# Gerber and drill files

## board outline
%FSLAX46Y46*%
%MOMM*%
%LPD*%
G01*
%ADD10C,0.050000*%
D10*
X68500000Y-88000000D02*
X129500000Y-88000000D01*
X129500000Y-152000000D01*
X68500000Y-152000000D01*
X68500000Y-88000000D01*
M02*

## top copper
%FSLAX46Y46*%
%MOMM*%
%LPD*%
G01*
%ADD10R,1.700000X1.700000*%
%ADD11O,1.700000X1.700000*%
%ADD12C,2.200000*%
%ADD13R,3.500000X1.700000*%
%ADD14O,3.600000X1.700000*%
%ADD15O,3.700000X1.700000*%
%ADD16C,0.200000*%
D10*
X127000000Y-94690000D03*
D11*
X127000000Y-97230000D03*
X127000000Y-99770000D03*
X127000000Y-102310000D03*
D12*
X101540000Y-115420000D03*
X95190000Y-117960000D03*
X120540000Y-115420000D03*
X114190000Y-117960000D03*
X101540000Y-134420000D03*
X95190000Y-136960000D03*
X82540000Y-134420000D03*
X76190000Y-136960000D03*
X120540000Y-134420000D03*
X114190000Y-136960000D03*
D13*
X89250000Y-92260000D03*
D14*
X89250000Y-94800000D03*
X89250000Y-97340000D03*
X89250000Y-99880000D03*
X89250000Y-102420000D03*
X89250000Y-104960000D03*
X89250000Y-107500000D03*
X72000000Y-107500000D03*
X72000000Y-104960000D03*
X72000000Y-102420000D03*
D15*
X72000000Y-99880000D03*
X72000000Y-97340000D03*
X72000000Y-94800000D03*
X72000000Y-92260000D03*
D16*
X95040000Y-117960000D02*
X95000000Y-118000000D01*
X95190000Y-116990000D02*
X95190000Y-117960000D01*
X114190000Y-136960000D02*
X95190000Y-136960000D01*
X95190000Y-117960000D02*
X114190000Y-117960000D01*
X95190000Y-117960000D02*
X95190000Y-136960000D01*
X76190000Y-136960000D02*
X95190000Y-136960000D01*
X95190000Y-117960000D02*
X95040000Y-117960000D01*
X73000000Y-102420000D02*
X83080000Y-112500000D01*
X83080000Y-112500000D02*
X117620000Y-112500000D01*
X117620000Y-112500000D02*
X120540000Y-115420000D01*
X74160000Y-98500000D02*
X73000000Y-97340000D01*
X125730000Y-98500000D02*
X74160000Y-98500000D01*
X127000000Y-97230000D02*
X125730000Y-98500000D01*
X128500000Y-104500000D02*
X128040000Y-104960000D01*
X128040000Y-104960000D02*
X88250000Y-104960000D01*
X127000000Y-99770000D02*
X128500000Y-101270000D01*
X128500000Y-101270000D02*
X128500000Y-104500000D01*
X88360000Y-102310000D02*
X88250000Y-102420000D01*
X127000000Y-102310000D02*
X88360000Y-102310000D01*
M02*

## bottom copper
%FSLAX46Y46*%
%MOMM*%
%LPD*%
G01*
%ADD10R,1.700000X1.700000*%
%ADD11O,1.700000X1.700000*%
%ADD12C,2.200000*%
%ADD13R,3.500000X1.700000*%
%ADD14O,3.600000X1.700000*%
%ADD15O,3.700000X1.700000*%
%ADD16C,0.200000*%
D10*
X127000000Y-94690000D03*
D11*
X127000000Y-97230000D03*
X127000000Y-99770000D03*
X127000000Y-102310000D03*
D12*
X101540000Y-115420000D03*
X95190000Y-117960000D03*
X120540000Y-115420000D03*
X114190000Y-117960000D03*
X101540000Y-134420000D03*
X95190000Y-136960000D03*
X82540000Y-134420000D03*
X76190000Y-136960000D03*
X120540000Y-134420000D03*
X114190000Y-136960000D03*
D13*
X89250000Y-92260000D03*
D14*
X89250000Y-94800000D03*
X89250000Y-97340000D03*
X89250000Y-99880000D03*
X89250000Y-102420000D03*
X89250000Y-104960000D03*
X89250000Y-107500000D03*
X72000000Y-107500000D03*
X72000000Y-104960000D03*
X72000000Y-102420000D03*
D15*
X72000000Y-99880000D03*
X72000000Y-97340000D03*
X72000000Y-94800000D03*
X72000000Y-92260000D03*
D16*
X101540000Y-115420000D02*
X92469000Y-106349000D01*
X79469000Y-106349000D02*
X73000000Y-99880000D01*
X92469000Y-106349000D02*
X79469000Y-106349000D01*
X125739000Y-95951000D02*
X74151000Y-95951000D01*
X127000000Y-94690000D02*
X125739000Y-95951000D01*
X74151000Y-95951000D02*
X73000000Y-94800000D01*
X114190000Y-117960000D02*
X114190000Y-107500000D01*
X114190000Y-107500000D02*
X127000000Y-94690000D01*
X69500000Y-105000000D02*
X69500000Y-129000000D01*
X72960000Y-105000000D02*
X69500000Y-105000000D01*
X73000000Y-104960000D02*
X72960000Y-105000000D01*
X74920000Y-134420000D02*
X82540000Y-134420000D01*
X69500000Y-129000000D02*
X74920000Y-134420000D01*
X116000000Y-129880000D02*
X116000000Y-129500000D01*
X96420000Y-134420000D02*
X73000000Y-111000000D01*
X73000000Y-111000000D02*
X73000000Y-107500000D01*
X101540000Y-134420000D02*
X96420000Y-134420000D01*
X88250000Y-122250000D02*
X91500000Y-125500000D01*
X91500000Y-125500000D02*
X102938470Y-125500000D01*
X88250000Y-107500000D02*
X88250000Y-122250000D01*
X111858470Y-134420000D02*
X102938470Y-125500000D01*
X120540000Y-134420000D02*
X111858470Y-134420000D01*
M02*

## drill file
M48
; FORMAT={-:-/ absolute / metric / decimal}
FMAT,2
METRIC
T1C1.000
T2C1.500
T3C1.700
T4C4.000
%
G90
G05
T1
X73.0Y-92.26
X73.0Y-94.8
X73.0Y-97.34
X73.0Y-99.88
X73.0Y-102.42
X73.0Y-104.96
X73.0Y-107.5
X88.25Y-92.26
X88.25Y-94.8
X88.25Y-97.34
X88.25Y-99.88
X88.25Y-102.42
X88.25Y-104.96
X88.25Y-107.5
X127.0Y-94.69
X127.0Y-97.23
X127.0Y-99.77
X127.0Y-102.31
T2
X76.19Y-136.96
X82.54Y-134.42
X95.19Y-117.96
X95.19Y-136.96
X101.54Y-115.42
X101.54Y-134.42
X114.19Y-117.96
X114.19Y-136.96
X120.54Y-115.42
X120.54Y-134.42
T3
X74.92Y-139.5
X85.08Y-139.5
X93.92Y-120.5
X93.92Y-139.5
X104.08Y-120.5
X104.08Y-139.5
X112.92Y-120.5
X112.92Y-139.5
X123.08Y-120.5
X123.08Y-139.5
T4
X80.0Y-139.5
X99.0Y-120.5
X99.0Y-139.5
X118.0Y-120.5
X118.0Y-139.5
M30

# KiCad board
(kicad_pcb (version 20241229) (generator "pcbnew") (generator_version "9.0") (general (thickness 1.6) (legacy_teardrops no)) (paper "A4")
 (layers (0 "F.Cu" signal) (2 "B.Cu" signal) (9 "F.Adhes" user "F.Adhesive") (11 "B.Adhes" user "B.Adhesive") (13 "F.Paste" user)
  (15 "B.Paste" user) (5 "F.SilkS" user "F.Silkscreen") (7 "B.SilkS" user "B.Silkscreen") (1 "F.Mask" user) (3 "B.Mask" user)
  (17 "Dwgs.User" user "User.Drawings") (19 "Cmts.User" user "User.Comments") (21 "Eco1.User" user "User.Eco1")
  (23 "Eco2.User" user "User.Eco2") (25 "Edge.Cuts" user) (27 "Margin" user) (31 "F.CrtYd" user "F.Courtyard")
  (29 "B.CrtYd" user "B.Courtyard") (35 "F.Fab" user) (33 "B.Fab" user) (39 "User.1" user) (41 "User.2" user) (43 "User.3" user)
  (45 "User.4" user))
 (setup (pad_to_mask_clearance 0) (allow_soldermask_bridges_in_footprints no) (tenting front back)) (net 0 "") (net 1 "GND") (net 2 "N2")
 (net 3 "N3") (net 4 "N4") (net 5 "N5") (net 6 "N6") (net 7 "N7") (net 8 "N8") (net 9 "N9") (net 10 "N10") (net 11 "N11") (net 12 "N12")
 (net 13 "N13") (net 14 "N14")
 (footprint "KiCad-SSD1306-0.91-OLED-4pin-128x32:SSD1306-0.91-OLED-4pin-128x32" (layer "F.Cu") (at 90.5 92.5)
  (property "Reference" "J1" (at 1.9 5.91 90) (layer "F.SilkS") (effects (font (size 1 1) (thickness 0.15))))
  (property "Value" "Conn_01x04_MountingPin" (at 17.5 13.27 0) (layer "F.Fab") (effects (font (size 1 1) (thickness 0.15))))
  (pad "1" thru_hole rect (at 36.5 2.19) (size 1.7 1.7) (drill 1) (layers "*.Cu" "*.Mask") (remove_unused_layers no) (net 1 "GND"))
  (pad "2" thru_hole oval (at 36.5 4.73) (size 1.7 1.7) (drill 1) (layers "*.Cu" "*.Mask") (remove_unused_layers no) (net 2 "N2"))
  (pad "3" thru_hole oval (at 36.5 7.27) (size 1.7 1.7) (drill 1) (layers "*.Cu" "*.Mask") (remove_unused_layers no) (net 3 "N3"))
  (pad "4" thru_hole oval (at 36.5 9.81) (size 1.7 1.7) (drill 1) (layers "*.Cu" "*.Mask") (remove_unused_layers no) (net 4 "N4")))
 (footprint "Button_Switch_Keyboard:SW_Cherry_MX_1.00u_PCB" (layer "F.Cu") (at 101.54 115.42)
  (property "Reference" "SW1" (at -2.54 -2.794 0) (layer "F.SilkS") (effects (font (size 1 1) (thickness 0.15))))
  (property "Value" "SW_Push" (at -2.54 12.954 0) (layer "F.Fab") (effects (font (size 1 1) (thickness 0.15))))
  (pad "" np_thru_hole circle (at -7.62 5.08) (size 1.7 1.7) (drill 1.7) (layers "*.Cu" "*.Mask"))
  (pad "" np_thru_hole circle (at -2.54 5.08) (size 4 4) (drill 4) (layers "*.Cu" "*.Mask"))
  (pad "" np_thru_hole circle (at 2.54 5.08) (size 1.7 1.7) (drill 1.7) (layers "*.Cu" "*.Mask"))
  (pad "1" thru_hole circle (at 0 0) (size 2.2 2.2) (drill 1.5) (layers "*.Cu" "*.Mask") (remove_unused_layers no) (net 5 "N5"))
  (pad "2" thru_hole circle (at -6.35 2.54) (size 2.2 2.2) (drill 1.5) (layers "*.Cu" "*.Mask") (remove_unused_layers no) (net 1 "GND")))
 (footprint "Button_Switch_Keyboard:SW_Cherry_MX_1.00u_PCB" (layer "F.Cu") (at 120.54 115.42)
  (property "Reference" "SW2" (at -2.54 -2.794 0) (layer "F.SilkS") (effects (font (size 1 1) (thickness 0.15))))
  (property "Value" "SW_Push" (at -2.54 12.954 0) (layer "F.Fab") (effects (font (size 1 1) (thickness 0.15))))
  (pad "" np_thru_hole circle (at -7.62 5.08) (size 1.7 1.7) (drill 1.7) (layers "*.Cu" "*.Mask"))
  (pad "" np_thru_hole circle (at -2.54 5.08) (size 4 4) (drill 4) (layers "*.Cu" "*.Mask"))
  (pad "" np_thru_hole circle (at 2.54 5.08) (size 1.7 1.7) (drill 1.7) (layers "*.Cu" "*.Mask"))
  (pad "1" thru_hole circle (at 0 0) (size 2.2 2.2) (drill 1.5) (layers "*.Cu" "*.Mask") (remove_unused_layers no) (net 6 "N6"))
  (pad "2" thru_hole circle (at -6.35 2.54) (size 2.2 2.2) (drill 1.5) (layers "*.Cu" "*.Mask") (remove_unused_layers no) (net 1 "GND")))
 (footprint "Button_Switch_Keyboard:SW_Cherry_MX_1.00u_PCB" (layer "F.Cu") (at 101.54 134.42)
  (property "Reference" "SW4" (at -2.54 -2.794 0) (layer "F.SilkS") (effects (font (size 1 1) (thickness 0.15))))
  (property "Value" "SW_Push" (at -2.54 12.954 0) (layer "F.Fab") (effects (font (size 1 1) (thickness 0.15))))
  (pad "" np_thru_hole circle (at -7.62 5.08) (size 1.7 1.7) (drill 1.7) (layers "*.Cu" "*.Mask"))
  (pad "" np_thru_hole circle (at -2.54 5.08) (size 4 4) (drill 4) (layers "*.Cu" "*.Mask"))
  (pad "" np_thru_hole circle (at 2.54 5.08) (size 1.7 1.7) (drill 1.7) (layers "*.Cu" "*.Mask"))
  (pad "1" thru_hole circle (at 0 0) (size 2.2 2.2) (drill 1.5) (layers "*.Cu" "*.Mask") (remove_unused_layers no) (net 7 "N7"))
  (pad "2" thru_hole circle (at -6.35 2.54) (size 2.2 2.2) (drill 1.5) (layers "*.Cu" "*.Mask") (remove_unused_layers no) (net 1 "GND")))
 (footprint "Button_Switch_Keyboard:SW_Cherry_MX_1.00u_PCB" (layer "F.Cu") (at 82.54 134.42)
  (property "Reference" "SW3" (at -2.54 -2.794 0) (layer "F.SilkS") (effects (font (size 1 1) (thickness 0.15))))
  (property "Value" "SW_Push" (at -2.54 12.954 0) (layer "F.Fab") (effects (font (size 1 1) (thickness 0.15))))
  (pad "" np_thru_hole circle (at -7.62 5.08) (size 1.7 1.7) (drill 1.7) (layers "*.Cu" "*.Mask"))
  (pad "" np_thru_hole circle (at -2.54 5.08) (size 4 4) (drill 4) (layers "*.Cu" "*.Mask"))
  (pad "" np_thru_hole circle (at 2.54 5.08) (size 1.7 1.7) (drill 1.7) (layers "*.Cu" "*.Mask"))
  (pad "1" thru_hole circle (at 0 0) (size 2.2 2.2) (drill 1.5) (layers "*.Cu" "*.Mask") (remove_unused_layers no) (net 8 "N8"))
  (pad "2" thru_hole circle (at -6.35 2.54) (size 2.2 2.2) (drill 1.5) (layers "*.Cu" "*.Mask") (remove_unused_layers no) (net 1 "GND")))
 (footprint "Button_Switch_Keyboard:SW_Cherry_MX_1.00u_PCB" (layer "F.Cu") (at 120.54 134.42)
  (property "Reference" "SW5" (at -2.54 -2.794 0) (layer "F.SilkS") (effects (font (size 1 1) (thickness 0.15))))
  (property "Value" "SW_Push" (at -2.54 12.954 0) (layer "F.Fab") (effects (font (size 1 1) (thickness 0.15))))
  (pad "" np_thru_hole circle (at -7.62 5.08) (size 1.7 1.7) (drill 1.7) (layers "*.Cu" "*.Mask"))
  (pad "" np_thru_hole circle (at -2.54 5.08) (size 4 4) (drill 4) (layers "*.Cu" "*.Mask"))
  (pad "" np_thru_hole circle (at 2.54 5.08) (size 1.7 1.7) (drill 1.7) (layers "*.Cu" "*.Mask"))
  (pad "1" thru_hole circle (at 0 0) (size 2.2 2.2) (drill 1.5) (layers "*.Cu" "*.Mask") (remove_unused_layers no) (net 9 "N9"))
  (pad "2" thru_hole circle (at -6.35 2.54) (size 2.2 2.2) (drill 1.5) (layers "*.Cu" "*.Mask") (remove_unused_layers no) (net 1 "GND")))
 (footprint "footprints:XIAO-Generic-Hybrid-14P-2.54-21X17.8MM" (layer "B.Cu") (at 80.625 99.88 180)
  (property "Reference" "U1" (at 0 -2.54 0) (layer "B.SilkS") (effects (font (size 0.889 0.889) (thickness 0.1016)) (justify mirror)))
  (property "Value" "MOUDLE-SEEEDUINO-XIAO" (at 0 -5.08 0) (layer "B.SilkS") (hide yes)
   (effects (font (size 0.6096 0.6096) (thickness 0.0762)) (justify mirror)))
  (pad "1" thru_hole rect (at -7.625 7.62 180) (size 3.5 1.7) (drill 1 (offset -1 0)) (layers "*.Cu" "*.Mask") (remove_unused_layers no)
   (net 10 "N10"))
  (pad "2" thru_hole oval (at -7.625 5.08 180) (size 3.6 1.7) (drill 1 (offset -1 0)) (layers "*.Cu" "*.Mask") (remove_unused_layers no)
   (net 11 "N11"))
  (pad "3" thru_hole oval (at -7.625 2.54 180) (size 3.6 1.7) (drill 1 (offset -1 0)) (layers "*.Cu" "*.Mask") (remove_unused_layers no)
   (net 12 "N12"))
  (pad "4" thru_hole oval (at -7.625 0 180) (size 3.6 1.7) (drill 1 (offset -1 0)) (layers "*.Cu" "*.Mask") (remove_unused_layers no)
   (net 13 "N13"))
  (pad "5" thru_hole oval (at -7.625 -2.54 180) (size 3.6 1.7) (drill 1 (offset -1 0)) (layers "*.Cu" "*.Mask") (remove_unused_layers no)
   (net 4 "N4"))
  (pad "6" thru_hole oval (at -7.625 -5.08) (size 3.6 1.7) (drill 1 (offset 1 0)) (layers "*.Cu" "*.Mask") (remove_unused_layers no)
   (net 3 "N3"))
  (pad "7" thru_hole oval (at -7.625 -7.62 180) (size 3.6 1.7) (drill 1 (offset -1 0)) (layers "*.Cu" "*.Mask") (remove_unused_layers no)
   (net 9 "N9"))
  (pad "8" thru_hole oval (at 7.625 -7.62 180) (size 3.6 1.7) (drill 1 (offset 1 0)) (layers "*.Cu" "*.Mask") (remove_unused_layers no)
   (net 7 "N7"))
  (pad "9" thru_hole oval (at 7.625 -5.08 180) (size 3.6 1.7) (drill 1 (offset 1 0)) (layers "*.Cu" "*.Mask") (remove_unused_layers no)
   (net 8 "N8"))
  (pad "10" thru_hole oval (at 7.625 -2.54 180) (size 3.6 1.7) (drill 1 (offset 1 0)) (layers "*.Cu" "*.Mask") (remove_unused_layers no)
   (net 6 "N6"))
  (pad "11" thru_hole oval (at 7.625 0 180) (size 3.7 1.7) (drill 1 (offset 1 0)) (layers "*.Cu" "*.Mask") (remove_unused_layers no)
   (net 5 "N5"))
  (pad "12" thru_hole oval (at 7.625 2.54 180) (size 3.7 1.7) (drill 1 (offset 1 0)) (layers "*.Cu" "*.Mask") (remove_unused_layers no)
   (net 2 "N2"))
  (pad "13" thru_hole oval (at 7.625 5.08 180) (size 3.7 1.7) (drill 1 (offset 1 0)) (layers "*.Cu" "*.Mask") (remove_unused_layers no)
   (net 1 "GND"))
  (pad "14" thru_hole oval (at 7.625 7.62 180) (size 3.7 1.7) (drill 1 (offset 1 0)) (layers "*.Cu" "*.Mask") (remove_unused_layers no)
   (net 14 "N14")))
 (gr_rect (start 68.5 88) (end 129.5 152) (stroke (width 0.05) (type default)) (fill no) (layer "Edge.Cuts"))
 (segment (start 101.54 115.42) (end 92.469 106.349) (width 0.2) (layer "B.Cu") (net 5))
 (segment (start 79.469 106.349) (end 73 99.88) (width 0.2) (layer "B.Cu") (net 5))
 (segment (start 92.469 106.349) (end 79.469 106.349) (width 0.2) (layer "B.Cu") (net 5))
 (segment (start 95.04 117.96) (end 95 118) (width 0.2) (layer "F.Cu") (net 1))
 (segment (start 95.19 116.99) (end 95.19 117.96) (width 0.2) (layer "F.Cu") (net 1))
 (segment (start 114.19 136.96) (end 95.19 136.96) (width 0.2) (layer "F.Cu") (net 1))
 (segment (start 95.19 117.96) (end 114.19 117.96) (width 0.2) (layer "F.Cu") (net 1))
 (segment (start 95.19 117.96) (end 95.19 136.96) (width 0.2) (layer "F.Cu") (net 1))
 (segment (start 76.19 136.96) (end 95.19 136.96) (width 0.2) (layer "F.Cu") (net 1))
 (segment (start 95.19 117.96) (end 95.04 117.96) (width 0.2) (layer "F.Cu") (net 1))
 (segment (start 125.739 95.951) (end 74.151 95.951) (width 0.2) (layer "B.Cu") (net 1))
 (segment (start 127 94.69) (end 125.739 95.951) (width 0.2) (layer "B.Cu") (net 1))
 (segment (start 74.151 95.951) (end 73 94.8) (width 0.2) (layer "B.Cu") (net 1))
 (segment (start 114.19 117.96) (end 114.19 107.5) (width 0.2) (layer "B.Cu") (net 1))
 (segment (start 114.19 107.5) (end 127 94.69) (width 0.2) (layer "B.Cu") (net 1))
 (segment (start 73 102.42) (end 83.08 112.5) (width 0.2) (layer "F.Cu") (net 6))
 (segment (start 83.08 112.5) (end 117.62 112.5) (width 0.2) (layer "F.Cu") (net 6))
 (segment (start 117.62 112.5) (end 120.54 115.42) (width 0.2) (layer "F.Cu") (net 6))
 (segment (start 69.5 105) (end 69.5 129) (width 0.2) (layer "B.Cu") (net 8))
 (segment (start 72.96 105) (end 69.5 105) (width 0.2) (layer "B.Cu") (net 8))
 (segment (start 73 104.96) (end 72.96 105) (width 0.2) (layer "B.Cu") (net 8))
 (segment (start 74.92 134.42) (end 82.54 134.42) (width 0.2) (layer "B.Cu") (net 8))
 (segment (start 69.5 129) (end 74.92 134.42) (width 0.2) (layer "B.Cu") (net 8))
 (segment (start 116 129.88) (end 116 129.5) (width 0.2) (layer "B.Cu") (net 7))
 (segment (start 96.42 134.42) (end 73 111) (width 0.2) (layer "B.Cu") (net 7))
 (segment (start 73 111) (end 73 107.5) (width 0.2) (layer "B.Cu") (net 7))
 (segment (start 101.54 134.42) (end 96.42 134.42) (width 0.2) (layer "B.Cu") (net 7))
 (segment (start 74.16 98.5) (end 73 97.34) (width 0.2) (layer "F.Cu") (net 2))
 (segment (start 125.73 98.5) (end 74.16 98.5) (width 0.2) (layer "F.Cu") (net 2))
 (segment (start 127 97.23) (end 125.73 98.5) (width 0.2) (layer "F.Cu") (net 2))
 (segment (start 128.5 104.5) (end 128.04 104.96) (width 0.2) (layer "F.Cu") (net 3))
 (segment (start 128.04 104.96) (end 88.25 104.96) (width 0.2) (layer "F.Cu") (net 3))
 (segment (start 127 99.77) (end 128.5 101.27) (width 0.2) (layer "F.Cu") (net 3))
 (segment (start 128.5 101.27) (end 128.5 104.5) (width 0.2) (layer "F.Cu") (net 3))
 (segment (start 88.36 102.31) (end 88.25 102.42) (width 0.2) (layer "F.Cu") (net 4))
 (segment (start 127 102.31) (end 88.36 102.31) (width 0.2) (layer "F.Cu") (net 4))
 (segment (start 88.25 122.25) (end 91.5 125.5) (width 0.2) (layer "B.Cu") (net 9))
 (segment (start 91.5 125.5) (end 102.93847 125.5) (width 0.2) (layer "B.Cu") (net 9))
 (segment (start 88.25 107.5) (end 88.25 122.25) (width 0.2) (layer "B.Cu") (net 9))
 (segment (start 111.85847 134.42) (end 102.93847 125.5) (width 0.2) (layer "B.Cu") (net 9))
 (segment (start 120.54 134.42) (end 111.85847 134.42) (width 0.2) (layer "B.Cu") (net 9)))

